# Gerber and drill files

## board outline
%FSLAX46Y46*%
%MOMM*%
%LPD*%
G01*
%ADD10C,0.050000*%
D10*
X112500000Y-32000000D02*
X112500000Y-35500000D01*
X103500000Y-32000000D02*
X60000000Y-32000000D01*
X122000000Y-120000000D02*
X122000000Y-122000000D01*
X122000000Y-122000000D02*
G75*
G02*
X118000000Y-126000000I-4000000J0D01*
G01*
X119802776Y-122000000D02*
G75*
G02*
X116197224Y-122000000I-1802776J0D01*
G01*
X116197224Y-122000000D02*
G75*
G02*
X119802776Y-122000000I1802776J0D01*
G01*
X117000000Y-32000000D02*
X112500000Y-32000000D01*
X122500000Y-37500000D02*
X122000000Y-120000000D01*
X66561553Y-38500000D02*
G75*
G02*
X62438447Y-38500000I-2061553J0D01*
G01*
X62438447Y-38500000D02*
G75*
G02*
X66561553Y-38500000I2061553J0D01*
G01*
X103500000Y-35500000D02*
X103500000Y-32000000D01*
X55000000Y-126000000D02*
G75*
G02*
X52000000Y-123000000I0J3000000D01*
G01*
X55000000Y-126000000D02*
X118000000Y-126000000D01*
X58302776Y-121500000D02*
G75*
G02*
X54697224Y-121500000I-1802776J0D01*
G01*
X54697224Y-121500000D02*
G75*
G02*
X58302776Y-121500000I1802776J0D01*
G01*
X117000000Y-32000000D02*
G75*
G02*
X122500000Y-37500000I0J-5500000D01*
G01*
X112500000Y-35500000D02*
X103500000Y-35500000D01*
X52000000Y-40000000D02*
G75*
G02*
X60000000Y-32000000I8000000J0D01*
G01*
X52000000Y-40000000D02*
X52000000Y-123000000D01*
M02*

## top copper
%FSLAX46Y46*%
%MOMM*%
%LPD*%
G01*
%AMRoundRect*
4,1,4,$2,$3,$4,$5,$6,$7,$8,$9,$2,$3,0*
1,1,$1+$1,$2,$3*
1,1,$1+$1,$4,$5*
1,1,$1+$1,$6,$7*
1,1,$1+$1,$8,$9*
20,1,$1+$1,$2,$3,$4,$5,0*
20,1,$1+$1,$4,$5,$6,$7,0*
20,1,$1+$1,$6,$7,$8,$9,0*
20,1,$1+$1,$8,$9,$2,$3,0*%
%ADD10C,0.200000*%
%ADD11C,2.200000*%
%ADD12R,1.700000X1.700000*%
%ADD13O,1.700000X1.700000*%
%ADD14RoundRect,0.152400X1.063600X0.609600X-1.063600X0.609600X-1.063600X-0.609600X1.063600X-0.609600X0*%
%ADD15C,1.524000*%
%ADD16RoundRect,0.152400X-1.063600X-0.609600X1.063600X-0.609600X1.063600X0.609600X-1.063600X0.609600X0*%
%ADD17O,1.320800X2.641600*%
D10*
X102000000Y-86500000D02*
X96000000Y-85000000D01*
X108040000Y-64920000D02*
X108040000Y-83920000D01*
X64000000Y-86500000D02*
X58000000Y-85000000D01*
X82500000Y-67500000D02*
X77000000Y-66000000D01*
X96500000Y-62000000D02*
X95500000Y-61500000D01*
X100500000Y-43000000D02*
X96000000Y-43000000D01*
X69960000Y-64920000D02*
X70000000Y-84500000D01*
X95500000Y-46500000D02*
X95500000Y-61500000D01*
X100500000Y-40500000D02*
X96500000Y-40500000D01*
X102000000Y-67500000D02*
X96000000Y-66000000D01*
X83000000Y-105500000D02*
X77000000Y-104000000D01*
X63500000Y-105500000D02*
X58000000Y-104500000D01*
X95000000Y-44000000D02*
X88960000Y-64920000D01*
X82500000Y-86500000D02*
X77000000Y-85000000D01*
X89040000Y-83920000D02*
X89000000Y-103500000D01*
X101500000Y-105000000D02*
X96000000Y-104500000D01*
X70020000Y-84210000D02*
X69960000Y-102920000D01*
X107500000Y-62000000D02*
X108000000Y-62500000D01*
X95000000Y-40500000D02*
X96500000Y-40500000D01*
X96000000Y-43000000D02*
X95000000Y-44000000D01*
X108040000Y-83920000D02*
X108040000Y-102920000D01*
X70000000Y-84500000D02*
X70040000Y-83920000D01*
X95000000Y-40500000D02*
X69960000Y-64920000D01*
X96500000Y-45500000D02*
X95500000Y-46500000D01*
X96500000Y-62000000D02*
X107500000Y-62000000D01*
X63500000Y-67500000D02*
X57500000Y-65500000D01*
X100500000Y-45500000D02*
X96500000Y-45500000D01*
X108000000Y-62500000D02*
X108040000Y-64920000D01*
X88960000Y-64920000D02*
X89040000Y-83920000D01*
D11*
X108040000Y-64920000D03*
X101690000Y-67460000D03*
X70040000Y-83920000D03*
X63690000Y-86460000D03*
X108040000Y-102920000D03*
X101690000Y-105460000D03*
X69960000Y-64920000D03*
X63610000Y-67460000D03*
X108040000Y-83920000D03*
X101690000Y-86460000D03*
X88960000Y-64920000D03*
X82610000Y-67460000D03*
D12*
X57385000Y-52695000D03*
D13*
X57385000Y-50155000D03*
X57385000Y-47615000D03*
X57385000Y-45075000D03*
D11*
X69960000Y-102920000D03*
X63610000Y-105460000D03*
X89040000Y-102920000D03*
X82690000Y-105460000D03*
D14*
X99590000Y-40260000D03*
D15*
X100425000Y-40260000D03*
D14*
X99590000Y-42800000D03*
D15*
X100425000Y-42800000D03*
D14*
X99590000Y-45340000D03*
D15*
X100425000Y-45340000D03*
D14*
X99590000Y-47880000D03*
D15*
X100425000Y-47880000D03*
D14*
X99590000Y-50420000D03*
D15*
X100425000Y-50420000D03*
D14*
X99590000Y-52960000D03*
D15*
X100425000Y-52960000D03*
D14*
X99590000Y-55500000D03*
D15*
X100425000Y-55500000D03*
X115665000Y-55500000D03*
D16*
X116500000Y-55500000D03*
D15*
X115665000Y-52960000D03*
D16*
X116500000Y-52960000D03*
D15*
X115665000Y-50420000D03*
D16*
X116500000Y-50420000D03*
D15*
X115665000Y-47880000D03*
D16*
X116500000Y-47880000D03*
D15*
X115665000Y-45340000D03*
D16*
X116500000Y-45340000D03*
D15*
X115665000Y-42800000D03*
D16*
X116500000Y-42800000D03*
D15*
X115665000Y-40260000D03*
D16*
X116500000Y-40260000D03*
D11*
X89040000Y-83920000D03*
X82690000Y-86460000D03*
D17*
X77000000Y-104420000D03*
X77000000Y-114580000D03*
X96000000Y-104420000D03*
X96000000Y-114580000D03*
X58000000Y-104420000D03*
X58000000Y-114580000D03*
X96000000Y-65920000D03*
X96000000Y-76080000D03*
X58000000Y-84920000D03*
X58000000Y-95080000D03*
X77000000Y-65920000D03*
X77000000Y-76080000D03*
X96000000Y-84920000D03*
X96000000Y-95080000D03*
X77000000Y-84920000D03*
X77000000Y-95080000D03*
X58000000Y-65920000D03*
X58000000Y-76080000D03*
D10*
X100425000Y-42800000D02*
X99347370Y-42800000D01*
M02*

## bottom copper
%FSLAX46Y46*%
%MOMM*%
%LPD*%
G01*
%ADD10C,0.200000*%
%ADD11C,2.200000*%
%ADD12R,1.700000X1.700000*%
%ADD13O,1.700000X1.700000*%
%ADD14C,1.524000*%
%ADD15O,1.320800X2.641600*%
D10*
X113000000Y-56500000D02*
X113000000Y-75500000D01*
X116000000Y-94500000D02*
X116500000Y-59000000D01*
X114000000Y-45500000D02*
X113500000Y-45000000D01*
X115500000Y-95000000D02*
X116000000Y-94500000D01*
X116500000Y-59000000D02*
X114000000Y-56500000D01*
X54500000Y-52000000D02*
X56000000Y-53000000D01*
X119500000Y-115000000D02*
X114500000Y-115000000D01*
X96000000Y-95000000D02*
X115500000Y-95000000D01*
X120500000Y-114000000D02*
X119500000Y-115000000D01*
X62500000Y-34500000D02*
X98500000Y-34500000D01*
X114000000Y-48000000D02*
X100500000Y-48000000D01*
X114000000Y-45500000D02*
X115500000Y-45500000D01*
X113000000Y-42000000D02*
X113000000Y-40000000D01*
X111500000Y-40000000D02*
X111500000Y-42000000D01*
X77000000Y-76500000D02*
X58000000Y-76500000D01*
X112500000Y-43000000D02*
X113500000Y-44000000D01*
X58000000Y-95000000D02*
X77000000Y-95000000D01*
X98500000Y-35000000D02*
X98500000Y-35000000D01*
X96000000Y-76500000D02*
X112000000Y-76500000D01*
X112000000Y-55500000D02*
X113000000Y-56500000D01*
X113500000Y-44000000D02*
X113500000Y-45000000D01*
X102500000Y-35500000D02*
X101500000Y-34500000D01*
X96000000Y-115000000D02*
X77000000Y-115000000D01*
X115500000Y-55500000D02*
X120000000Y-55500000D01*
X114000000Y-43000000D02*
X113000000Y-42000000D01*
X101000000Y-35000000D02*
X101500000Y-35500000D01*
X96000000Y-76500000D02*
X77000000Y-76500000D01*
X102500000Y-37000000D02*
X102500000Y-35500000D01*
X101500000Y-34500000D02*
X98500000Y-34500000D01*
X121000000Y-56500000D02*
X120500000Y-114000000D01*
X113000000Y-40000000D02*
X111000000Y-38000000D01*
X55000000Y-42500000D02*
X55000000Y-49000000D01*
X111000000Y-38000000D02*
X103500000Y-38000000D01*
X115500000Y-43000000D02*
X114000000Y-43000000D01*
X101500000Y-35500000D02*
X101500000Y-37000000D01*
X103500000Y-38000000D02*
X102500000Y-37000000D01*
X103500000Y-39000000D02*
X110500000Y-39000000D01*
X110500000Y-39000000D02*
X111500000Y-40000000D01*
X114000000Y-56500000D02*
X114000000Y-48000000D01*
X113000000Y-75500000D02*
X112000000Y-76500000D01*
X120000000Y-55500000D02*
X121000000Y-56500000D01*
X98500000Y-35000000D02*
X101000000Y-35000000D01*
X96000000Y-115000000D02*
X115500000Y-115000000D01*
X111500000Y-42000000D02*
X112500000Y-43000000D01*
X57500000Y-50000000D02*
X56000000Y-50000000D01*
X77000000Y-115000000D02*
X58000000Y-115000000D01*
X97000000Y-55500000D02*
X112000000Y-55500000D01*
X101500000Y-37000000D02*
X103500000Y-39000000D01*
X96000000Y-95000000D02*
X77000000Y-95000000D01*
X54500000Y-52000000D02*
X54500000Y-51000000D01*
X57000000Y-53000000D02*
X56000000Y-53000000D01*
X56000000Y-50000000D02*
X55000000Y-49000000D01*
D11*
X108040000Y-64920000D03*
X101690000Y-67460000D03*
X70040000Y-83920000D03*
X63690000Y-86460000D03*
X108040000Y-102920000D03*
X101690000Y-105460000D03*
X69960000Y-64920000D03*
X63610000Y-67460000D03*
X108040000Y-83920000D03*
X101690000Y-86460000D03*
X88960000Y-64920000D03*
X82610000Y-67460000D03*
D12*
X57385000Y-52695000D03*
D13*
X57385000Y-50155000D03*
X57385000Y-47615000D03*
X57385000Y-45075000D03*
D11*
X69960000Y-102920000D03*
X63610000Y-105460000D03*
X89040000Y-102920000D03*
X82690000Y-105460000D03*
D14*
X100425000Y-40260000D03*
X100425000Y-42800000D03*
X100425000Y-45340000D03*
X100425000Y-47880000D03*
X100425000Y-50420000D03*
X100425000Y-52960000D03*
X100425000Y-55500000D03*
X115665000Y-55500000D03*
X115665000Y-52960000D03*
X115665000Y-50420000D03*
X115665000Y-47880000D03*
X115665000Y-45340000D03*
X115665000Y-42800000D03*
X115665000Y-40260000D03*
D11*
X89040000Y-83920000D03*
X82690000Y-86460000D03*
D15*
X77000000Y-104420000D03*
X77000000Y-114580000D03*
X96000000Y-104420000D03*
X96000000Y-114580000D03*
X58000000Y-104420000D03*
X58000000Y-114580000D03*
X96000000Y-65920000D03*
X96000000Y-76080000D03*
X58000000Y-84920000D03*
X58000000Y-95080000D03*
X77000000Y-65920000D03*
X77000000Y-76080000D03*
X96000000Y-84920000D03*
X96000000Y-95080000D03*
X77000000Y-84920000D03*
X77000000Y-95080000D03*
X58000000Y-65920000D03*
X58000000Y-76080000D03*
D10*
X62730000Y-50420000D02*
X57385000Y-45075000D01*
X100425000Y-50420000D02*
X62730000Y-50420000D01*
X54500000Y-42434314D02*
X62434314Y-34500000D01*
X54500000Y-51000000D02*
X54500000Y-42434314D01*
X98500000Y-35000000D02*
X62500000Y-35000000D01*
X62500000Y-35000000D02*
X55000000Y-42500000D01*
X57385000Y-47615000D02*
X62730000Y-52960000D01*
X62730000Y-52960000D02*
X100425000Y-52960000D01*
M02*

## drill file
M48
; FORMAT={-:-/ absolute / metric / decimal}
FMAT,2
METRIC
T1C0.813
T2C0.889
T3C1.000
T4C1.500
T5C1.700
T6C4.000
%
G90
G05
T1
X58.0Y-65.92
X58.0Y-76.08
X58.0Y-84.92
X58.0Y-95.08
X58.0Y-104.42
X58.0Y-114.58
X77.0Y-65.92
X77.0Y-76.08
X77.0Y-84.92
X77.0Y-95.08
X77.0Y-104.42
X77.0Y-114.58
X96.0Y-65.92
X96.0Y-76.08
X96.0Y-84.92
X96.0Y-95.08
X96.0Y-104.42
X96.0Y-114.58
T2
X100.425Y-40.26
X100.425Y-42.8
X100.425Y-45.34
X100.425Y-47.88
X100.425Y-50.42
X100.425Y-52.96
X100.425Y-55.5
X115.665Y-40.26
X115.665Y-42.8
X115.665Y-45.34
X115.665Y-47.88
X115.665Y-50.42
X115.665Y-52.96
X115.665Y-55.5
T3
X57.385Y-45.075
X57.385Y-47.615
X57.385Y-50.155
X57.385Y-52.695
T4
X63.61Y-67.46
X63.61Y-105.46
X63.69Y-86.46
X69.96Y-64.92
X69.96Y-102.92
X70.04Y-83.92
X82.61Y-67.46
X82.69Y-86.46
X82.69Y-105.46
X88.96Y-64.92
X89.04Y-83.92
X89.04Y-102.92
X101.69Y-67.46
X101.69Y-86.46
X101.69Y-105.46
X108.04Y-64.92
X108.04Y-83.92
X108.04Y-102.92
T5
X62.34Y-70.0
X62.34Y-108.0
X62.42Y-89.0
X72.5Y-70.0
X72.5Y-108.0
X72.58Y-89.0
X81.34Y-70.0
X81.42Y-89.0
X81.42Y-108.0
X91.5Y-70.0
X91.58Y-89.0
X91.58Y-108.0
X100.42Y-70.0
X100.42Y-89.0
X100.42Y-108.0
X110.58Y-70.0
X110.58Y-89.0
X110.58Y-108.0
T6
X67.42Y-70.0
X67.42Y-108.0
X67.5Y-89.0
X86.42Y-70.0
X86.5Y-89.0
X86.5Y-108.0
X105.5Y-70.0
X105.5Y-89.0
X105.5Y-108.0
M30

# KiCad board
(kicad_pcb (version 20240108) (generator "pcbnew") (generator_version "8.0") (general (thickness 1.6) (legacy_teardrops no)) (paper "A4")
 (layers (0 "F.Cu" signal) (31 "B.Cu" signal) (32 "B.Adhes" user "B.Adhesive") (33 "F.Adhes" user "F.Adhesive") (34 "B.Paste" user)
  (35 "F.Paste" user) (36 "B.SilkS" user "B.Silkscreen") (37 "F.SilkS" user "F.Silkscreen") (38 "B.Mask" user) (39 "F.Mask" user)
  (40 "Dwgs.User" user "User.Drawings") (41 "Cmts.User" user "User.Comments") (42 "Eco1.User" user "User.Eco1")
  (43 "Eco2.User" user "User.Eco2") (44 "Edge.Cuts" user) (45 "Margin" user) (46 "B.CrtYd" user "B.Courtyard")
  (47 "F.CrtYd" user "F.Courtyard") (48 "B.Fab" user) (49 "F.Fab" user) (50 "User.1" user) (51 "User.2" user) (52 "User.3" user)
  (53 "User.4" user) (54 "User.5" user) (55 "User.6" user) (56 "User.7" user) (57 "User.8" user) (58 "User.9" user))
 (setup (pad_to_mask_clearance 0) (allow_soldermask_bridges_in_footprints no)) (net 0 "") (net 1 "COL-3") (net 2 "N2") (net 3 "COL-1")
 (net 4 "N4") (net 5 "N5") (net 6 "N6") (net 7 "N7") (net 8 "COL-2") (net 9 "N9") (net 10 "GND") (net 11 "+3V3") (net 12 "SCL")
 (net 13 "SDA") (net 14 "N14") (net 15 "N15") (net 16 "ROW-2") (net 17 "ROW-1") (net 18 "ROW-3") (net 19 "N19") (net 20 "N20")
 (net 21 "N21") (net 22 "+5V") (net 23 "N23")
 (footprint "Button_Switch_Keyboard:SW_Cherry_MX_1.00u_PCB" (layer "F.Cu") (at 108.04 64.92)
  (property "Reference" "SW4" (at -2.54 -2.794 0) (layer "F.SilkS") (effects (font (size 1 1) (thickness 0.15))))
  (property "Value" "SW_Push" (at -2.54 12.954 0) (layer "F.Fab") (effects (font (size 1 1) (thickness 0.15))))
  (pad "" np_thru_hole circle (at -7.62 5.08) (size 1.7 1.7) (drill 1.7) (layers "*.Cu" "*.Mask"))
  (pad "" np_thru_hole circle (at -2.54 5.08) (size 4 4) (drill 4) (layers "*.Cu" "*.Mask"))
  (pad "" np_thru_hole circle (at 2.54 5.08) (size 1.7 1.7) (drill 1.7) (layers "*.Cu" "*.Mask"))
  (pad "1" thru_hole circle (at 0 0) (size 2.2 2.2) (drill 1.5) (layers "*.Cu" "*.Mask") (remove_unused_layers no) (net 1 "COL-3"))
  (pad "2" thru_hole circle (at -6.35 2.54) (size 2.2 2.2) (drill 1.5) (layers "*.Cu" "*.Mask") (remove_unused_layers no) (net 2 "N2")))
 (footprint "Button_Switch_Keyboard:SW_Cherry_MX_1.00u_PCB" (layer "F.Cu") (at 70.04 83.92)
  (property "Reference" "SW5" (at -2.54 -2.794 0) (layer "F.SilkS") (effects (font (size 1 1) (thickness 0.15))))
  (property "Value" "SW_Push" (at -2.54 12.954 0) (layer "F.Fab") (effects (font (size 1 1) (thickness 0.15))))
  (pad "" np_thru_hole circle (at -7.62 5.08) (size 1.7 1.7) (drill 1.7) (layers "*.Cu" "*.Mask"))
  (pad "" np_thru_hole circle (at -2.54 5.08) (size 4 4) (drill 4) (layers "*.Cu" "*.Mask"))
  (pad "" np_thru_hole circle (at 2.54 5.08) (size 1.7 1.7) (drill 1.7) (layers "*.Cu" "*.Mask"))
  (pad "1" thru_hole circle (at 0 0) (size 2.2 2.2) (drill 1.5) (layers "*.Cu" "*.Mask") (remove_unused_layers no) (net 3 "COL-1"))
  (pad "2" thru_hole circle (at -6.35 2.54) (size 2.2 2.2) (drill 1.5) (layers "*.Cu" "*.Mask") (remove_unused_layers no) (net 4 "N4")))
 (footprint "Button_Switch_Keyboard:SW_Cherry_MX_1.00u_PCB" (layer "F.Cu") (at 108.04 102.92)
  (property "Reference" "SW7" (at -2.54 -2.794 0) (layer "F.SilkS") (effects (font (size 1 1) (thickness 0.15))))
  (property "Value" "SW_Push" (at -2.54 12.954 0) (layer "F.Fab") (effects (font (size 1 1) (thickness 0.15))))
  (pad "" np_thru_hole circle (at -7.62 5.08) (size 1.7 1.7) (drill 1.7) (layers "*.Cu" "*.Mask"))
  (pad "" np_thru_hole circle (at -2.54 5.08) (size 4 4) (drill 4) (layers "*.Cu" "*.Mask"))
  (pad "" np_thru_hole circle (at 2.54 5.08) (size 1.7 1.7) (drill 1.7) (layers "*.Cu" "*.Mask"))
  (pad "1" thru_hole circle (at 0 0) (size 2.2 2.2) (drill 1.5) (layers "*.Cu" "*.Mask") (remove_unused_layers no) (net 1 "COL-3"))
  (pad "2" thru_hole circle (at -6.35 2.54) (size 2.2 2.2) (drill 1.5) (layers "*.Cu" "*.Mask") (remove_unused_layers no) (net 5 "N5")))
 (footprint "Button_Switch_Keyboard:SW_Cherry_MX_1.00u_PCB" (layer "F.Cu") (at 69.96 64.92)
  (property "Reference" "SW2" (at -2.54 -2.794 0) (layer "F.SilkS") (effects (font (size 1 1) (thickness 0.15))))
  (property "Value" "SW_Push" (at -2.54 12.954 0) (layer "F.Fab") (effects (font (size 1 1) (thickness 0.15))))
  (pad "" np_thru_hole circle (at -7.62 5.08) (size 1.7 1.7) (drill 1.7) (layers "*.Cu" "*.Mask"))
  (pad "" np_thru_hole circle (at -2.54 5.08) (size 4 4) (drill 4) (layers "*.Cu" "*.Mask"))
  (pad "" np_thru_hole circle (at 2.54 5.08) (size 1.7 1.7) (drill 1.7) (layers "*.Cu" "*.Mask"))
  (pad "1" thru_hole circle (at 0 0) (size 2.2 2.2) (drill 1.5) (layers "*.Cu" "*.Mask") (remove_unused_layers no) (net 3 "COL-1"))
  (pad "2" thru_hole circle (at -6.35 2.54) (size 2.2 2.2) (drill 1.5) (layers "*.Cu" "*.Mask") (remove_unused_layers no) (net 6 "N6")))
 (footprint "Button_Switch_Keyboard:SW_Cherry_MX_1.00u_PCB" (layer "F.Cu") (at 108.04 83.92)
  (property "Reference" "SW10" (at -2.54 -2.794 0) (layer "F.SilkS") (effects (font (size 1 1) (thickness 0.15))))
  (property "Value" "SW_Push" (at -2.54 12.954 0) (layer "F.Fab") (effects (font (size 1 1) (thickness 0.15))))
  (pad "" np_thru_hole circle (at -7.62 5.08) (size 1.7 1.7) (drill 1.7) (layers "*.Cu" "*.Mask"))
  (pad "" np_thru_hole circle (at -2.54 5.08) (size 4 4) (drill 4) (layers "*.Cu" "*.Mask"))
  (pad "" np_thru_hole circle (at 2.54 5.08) (size 1.7 1.7) (drill 1.7) (layers "*.Cu" "*.Mask"))
  (pad "1" thru_hole circle (at 0 0) (size 2.2 2.2) (drill 1.5) (layers "*.Cu" "*.Mask") (remove_unused_layers no) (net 1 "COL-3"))
  (pad "2" thru_hole circle (at -6.35 2.54) (size 2.2 2.2) (drill 1.5) (layers "*.Cu" "*.Mask") (remove_unused_layers no) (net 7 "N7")))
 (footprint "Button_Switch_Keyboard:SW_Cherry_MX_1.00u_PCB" (layer "F.Cu") (at 88.96 64.92)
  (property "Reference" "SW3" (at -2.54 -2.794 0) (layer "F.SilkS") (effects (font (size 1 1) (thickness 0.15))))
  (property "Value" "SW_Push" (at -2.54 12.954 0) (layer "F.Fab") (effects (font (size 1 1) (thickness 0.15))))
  (pad "" np_thru_hole circle (at -7.62 5.08) (size 1.7 1.7) (drill 1.7) (layers "*.Cu" "*.Mask"))
  (pad "" np_thru_hole circle (at -2.54 5.08) (size 4 4) (drill 4) (layers "*.Cu" "*.Mask"))
  (pad "" np_thru_hole circle (at 2.54 5.08) (size 1.7 1.7) (drill 1.7) (layers "*.Cu" "*.Mask"))
  (pad "1" thru_hole circle (at 0 0) (size 2.2 2.2) (drill 1.5) (layers "*.Cu" "*.Mask") (remove_unused_layers no) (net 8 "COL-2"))
  (pad "2" thru_hole circle (at -6.35 2.54) (size 2.2 2.2) (drill 1.5) (layers "*.Cu" "*.Mask") (remove_unused_layers no) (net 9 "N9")))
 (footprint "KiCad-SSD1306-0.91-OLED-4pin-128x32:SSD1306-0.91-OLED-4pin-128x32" (layer "F.Cu") (at 93.885 54.885 180)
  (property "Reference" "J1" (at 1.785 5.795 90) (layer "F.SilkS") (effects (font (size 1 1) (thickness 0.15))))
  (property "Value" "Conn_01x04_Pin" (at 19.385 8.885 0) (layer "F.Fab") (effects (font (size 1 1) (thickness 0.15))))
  (pad "1" thru_hole rect (at 36.5 2.19 180) (size 1.7 1.7) (drill 1) (layers "*.Cu" "*.Mask") (remove_unused_layers no) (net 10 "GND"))
  (pad "2" thru_hole oval (at 36.5 4.73 180) (size 1.7 1.7) (drill 1) (layers "*.Cu" "*.Mask") (remove_unused_layers no) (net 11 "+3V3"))
  (pad "3" thru_hole oval (at 36.5 7.27 180) (size 1.7 1.7) (drill 1) (layers "*.Cu" "*.Mask") (remove_unused_layers no) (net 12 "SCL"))
  (pad "4" thru_hole oval (at 36.5 9.81 180) (size 1.7 1.7) (drill 1) (layers "*.Cu" "*.Mask") (remove_unused_layers no) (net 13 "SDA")))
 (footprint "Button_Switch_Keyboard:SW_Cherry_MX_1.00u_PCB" (layer "F.Cu") (at 69.96 102.92)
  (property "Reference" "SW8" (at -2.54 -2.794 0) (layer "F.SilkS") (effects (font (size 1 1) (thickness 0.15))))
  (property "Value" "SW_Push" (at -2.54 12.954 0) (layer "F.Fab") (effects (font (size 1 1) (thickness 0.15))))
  (pad "" np_thru_hole circle (at -7.62 5.08) (size 1.7 1.7) (drill 1.7) (layers "*.Cu" "*.Mask"))
  (pad "" np_thru_hole circle (at -2.54 5.08) (size 4 4) (drill 4) (layers "*.Cu" "*.Mask"))
  (pad "" np_thru_hole circle (at 2.54 5.08) (size 1.7 1.7) (drill 1.7) (layers "*.Cu" "*.Mask"))
  (pad "1" thru_hole circle (at 0 0) (size 2.2 2.2) (drill 1.5) (layers "*.Cu" "*.Mask") (remove_unused_layers no) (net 3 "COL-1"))
  (pad "2" thru_hole circle (at -6.35 2.54) (size 2.2 2.2) (drill 1.5) (layers "*.Cu" "*.Mask") (remove_unused_layers no) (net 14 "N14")))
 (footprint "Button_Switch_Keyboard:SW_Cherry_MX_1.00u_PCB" (layer "F.Cu") (at 89.04 102.92)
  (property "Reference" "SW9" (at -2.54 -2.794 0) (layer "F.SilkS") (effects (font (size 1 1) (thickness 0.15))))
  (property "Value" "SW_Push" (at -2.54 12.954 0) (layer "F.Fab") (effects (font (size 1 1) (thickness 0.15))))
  (pad "" np_thru_hole circle (at -7.62 5.08) (size 1.7 1.7) (drill 1.7) (layers "*.Cu" "*.Mask"))
  (pad "" np_thru_hole circle (at -2.54 5.08) (size 4 4) (drill 4) (layers "*.Cu" "*.Mask"))
  (pad "" np_thru_hole circle (at 2.54 5.08) (size 1.7 1.7) (drill 1.7) (layers "*.Cu" "*.Mask"))
  (pad "1" thru_hole circle (at 0 0) (size 2.2 2.2) (drill 1.5) (layers "*.Cu" "*.Mask") (remove_unused_layers no) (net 8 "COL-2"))
  (pad "2" thru_hole circle (at -6.35 2.54) (size 2.2 2.2) (drill 1.5) (layers "*.Cu" "*.Mask") (remove_unused_layers no) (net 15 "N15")))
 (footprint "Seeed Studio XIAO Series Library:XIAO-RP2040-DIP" (layer "F.Cu") (at 108.045 47.88)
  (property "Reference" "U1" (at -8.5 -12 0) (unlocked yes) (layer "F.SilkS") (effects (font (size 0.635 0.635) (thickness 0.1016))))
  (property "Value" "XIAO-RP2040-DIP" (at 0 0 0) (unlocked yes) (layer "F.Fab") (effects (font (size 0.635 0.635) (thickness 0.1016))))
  (pad "1" smd roundrect (at -8.455 -7.62 180) (size 2.432 1.524) (layers "F.Cu" "F.Mask") (roundrect_rratio 0.1) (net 3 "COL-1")
   (thermal_bridge_angle 45))
  (pad "1" thru_hole circle (at -7.62 -7.62 180) (size 1.524 1.524) (drill 0.889) (layers "*.Cu" "*.Mask") (remove_unused_layers no)
   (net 3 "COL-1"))
  (pad "2" smd roundrect (at -8.455 -5.08 180) (size 2.432 1.524) (layers "F.Cu" "F.Mask") (roundrect_rratio 0.1) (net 8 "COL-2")
   (thermal_bridge_angle 45))
  (pad "2" thru_hole circle (at -7.62 -5.08 180) (size 1.524 1.524) (drill 0.889) (layers "*.Cu" "*.Mask") (remove_unused_layers no)
   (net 8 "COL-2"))
  (pad "3" smd roundrect (at -8.455 -2.54 180) (size 2.432 1.524) (layers "F.Cu" "F.Mask") (roundrect_rratio 0.1) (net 1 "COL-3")
   (thermal_bridge_angle 45))
  (pad "3" thru_hole circle (at -7.62 -2.54 180) (size 1.524 1.524) (drill 0.889) (layers "*.Cu" "*.Mask") (remove_unused_layers no)
   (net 1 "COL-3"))
  (pad "4" smd roundrect (at -8.455 0 180) (size 2.432 1.524) (layers "F.Cu" "F.Mask") (roundrect_rratio 0.1) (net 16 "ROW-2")
   (thermal_bridge_angle 45))
  (pad "4" thru_hole circle (at -7.62 0 180) (size 1.524 1.524) (drill 0.889) (layers "*.Cu" "*.Mask") (remove_unused_layers no)
   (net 16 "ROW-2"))
  (pad "5" smd roundrect (at -8.455 2.54 180) (size 2.432 1.524) (layers "F.Cu" "F.Mask") (roundrect_rratio 0.1) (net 13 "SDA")
   (thermal_bridge_angle 45))
  (pad "5" thru_hole circle (at -7.62 2.54 180) (size 1.524 1.524) (drill 0.889) (layers "*.Cu" "*.Mask") (remove_unused_layers no)
   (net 13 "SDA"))
  (pad "6" smd roundrect (at -8.455 5.08 180) (size 2.432 1.524) (layers "F.Cu" "F.Mask") (roundrect_rratio 0.1) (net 12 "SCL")
   (thermal_bridge_angle 45))
  (pad "6" thru_hole circle (at -7.62 5.08 180) (size 1.524 1.524) (drill 0.889) (layers "*.Cu" "*.Mask") (remove_unused_layers no)
   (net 12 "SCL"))
  (pad "7" smd roundrect (at -8.455 7.62 180) (size 2.432 1.524) (layers "F.Cu" "F.Mask") (roundrect_rratio 0.1) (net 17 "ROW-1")
   (thermal_bridge_angle 45))
  (pad "7" thru_hole circle (at -7.62 7.62 180) (size 1.524 1.524) (drill 0.889) (layers "*.Cu" "*.Mask") (remove_unused_layers no)
   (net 17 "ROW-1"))
  (pad "8" thru_hole circle (at 7.62 7.62) (size 1.524 1.524) (drill 0.889) (layers "*.Cu" "*.Mask") (remove_unused_layers no)
   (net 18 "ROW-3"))
  (pad "8" smd roundrect (at 8.455 7.62) (size 2.432 1.524) (layers "F.Cu" "F.Mask") (roundrect_rratio 0.1) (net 18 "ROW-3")
   (thermal_bridge_angle 45))
  (pad "9" thru_hole circle (at 7.62 5.08) (size 1.524 1.524) (drill 0.889) (layers "*.Cu" "*.Mask") (remove_unused_layers no)
   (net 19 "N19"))
  (pad "9" smd roundrect (at 8.455 5.08) (size 2.432 1.524) (layers "F.Cu" "F.Mask") (roundrect_rratio 0.1) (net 19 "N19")
   (thermal_bridge_angle 45))
  (pad "10" thru_hole circle (at 7.62 2.54) (size 1.524 1.524) (drill 0.889) (layers "*.Cu" "*.Mask") (remove_unused_layers no)
   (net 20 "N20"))
  (pad "10" smd roundrect (at 8.455 2.54) (size 2.432 1.524) (layers "F.Cu" "F.Mask") (roundrect_rratio 0.1) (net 20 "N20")
   (thermal_bridge_angle 45))
  (pad "11" thru_hole circle (at 7.62 0) (size 1.524 1.524) (drill 0.889) (layers "*.Cu" "*.Mask") (remove_unused_layers no) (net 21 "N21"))
  (pad "11" smd roundrect (at 8.455 0) (size 2.432 1.524) (layers "F.Cu" "F.Mask") (roundrect_rratio 0.1) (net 21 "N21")
   (thermal_bridge_angle 45))
  (pad "12" thru_hole circle (at 7.62 -2.54) (size 1.524 1.524) (drill 0.889) (layers "*.Cu" "*.Mask") (remove_unused_layers no)
   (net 11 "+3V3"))
  (pad "12" smd roundrect (at 8.455 -2.54) (size 2.432 1.524) (layers "F.Cu" "F.Mask") (roundrect_rratio 0.1) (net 11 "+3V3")
   (thermal_bridge_angle 45))
  (pad "13" thru_hole circle (at 7.62 -5.08) (size 1.524 1.524) (drill 0.889) (layers "*.Cu" "*.Mask") (remove_unused_layers no)
   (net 10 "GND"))
  (pad "13" smd roundrect (at 8.455 -5.08) (size 2.432 1.524) (layers "F.Cu" "F.Mask") (roundrect_rratio 0.1) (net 10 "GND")
   (thermal_bridge_angle 45))
  (pad "14" thru_hole circle (at 7.62 -7.62) (size 1.524 1.524) (drill 0.889) (layers "*.Cu" "*.Mask") (remove_unused_layers no)
   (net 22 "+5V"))
  (pad "14" smd roundrect (at 8.455 -7.62) (size 2.432 1.524) (layers "F.Cu" "F.Mask") (roundrect_rratio 0.1) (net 22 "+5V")
   (thermal_bridge_angle 45)))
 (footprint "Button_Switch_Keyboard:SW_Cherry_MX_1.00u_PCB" (layer "F.Cu") (at 89.04 83.92)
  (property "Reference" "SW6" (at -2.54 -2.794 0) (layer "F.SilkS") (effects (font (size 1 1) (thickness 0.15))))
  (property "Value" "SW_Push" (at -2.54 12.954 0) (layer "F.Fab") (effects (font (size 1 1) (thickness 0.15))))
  (pad "" np_thru_hole circle (at -7.62 5.08) (size 1.7 1.7) (drill 1.7) (layers "*.Cu" "*.Mask"))
  (pad "" np_thru_hole circle (at -2.54 5.08) (size 4 4) (drill 4) (layers "*.Cu" "*.Mask"))
  (pad "" np_thru_hole circle (at 2.54 5.08) (size 1.7 1.7) (drill 1.7) (layers "*.Cu" "*.Mask"))
  (pad "1" thru_hole circle (at 0 0) (size 2.2 2.2) (drill 1.5) (layers "*.Cu" "*.Mask") (remove_unused_layers no) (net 8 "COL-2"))
  (pad "2" thru_hole circle (at -6.35 2.54) (size 2.2 2.2) (drill 1.5) (layers "*.Cu" "*.Mask") (remove_unused_layers no) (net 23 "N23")))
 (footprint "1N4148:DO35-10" (layer "B.Cu") (at 77 109.5 90)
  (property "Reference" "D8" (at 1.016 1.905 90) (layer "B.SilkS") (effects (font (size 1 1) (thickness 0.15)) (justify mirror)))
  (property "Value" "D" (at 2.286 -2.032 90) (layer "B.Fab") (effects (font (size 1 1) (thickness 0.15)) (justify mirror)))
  (pad "A" thru_hole oval (at 5.08 0 90) (size 2.6416 1.3208) (drill 0.8128) (layers "*.Cu" "*.Mask") (remove_unused_layers no)
   (solder_mask_margin 0.102))
  (pad "C" thru_hole oval (at -5.08 0 90) (size 2.6416 1.3208) (drill 0.8128) (layers "*.Cu" "*.Mask") (remove_unused_layers no)
   (solder_mask_margin 0.102)))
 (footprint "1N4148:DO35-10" (layer "B.Cu") (at 96 109.5 90)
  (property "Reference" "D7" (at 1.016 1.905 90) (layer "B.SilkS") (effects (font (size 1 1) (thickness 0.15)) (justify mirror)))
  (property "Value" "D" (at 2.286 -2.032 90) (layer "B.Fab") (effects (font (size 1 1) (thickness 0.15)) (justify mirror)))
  (pad "A" thru_hole oval (at 5.08 0 90) (size 2.6416 1.3208) (drill 0.8128) (layers "*.Cu" "*.Mask") (remove_unused_layers no)
   (solder_mask_margin 0.102))
  (pad "C" thru_hole oval (at -5.08 0 90) (size 2.6416 1.3208) (drill 0.8128) (layers "*.Cu" "*.Mask") (remove_unused_layers no)
   (solder_mask_margin 0.102)))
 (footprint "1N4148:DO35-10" (layer "B.Cu") (at 58 109.5 90)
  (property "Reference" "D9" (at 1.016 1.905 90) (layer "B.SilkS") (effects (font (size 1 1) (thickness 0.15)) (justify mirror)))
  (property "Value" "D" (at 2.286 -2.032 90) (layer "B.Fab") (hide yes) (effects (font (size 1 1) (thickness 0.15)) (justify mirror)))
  (pad "A" thru_hole oval (at 5.08 0 90) (size 2.6416 1.3208) (drill 0.8128) (layers "*.Cu" "*.Mask") (remove_unused_layers no)
   (solder_mask_margin 0.102))
  (pad "C" thru_hole oval (at -5.08 0 90) (size 2.6416 1.3208) (drill 0.8128) (layers "*.Cu" "*.Mask") (remove_unused_layers no)
   (solder_mask_margin 0.102)))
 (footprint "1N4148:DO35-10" (layer "B.Cu") (at 96 71 90)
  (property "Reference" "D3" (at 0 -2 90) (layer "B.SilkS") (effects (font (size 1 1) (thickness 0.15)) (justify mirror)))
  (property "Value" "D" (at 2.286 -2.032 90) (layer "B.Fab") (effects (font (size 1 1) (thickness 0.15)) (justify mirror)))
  (pad "A" thru_hole oval (at 5.08 0 90) (size 2.6416 1.3208) (drill 0.8128) (layers "*.Cu" "*.Mask") (remove_unused_layers no)
   (solder_mask_margin 0.102))
  (pad "C" thru_hole oval (at -5.08 0 90) (size 2.6416 1.3208) (drill 0.8128) (layers "*.Cu" "*.Mask") (remove_unused_layers no)
   (solder_mask_margin 0.102)))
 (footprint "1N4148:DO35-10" (layer "B.Cu") (at 58 90 90)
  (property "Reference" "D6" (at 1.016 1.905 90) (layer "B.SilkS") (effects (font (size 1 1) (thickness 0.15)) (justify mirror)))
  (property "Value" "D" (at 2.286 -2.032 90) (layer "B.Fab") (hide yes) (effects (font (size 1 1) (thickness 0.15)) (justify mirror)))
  (pad "A" thru_hole oval (at 5.08 0 90) (size 2.6416 1.3208) (drill 0.8128) (layers "*.Cu" "*.Mask") (remove_unused_layers no)
   (solder_mask_margin 0.102))
  (pad "C" thru_hole oval (at -5.08 0 90) (size 2.6416 1.3208) (drill 0.8128) (layers "*.Cu" "*.Mask") (remove_unused_layers no)
   (solder_mask_margin 0.102)))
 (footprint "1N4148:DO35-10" (layer "B.Cu") (at 77 71 90)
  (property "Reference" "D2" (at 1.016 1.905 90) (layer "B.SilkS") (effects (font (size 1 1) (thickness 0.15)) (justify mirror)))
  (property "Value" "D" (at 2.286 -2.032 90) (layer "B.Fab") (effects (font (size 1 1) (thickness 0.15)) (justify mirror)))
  (pad "A" thru_hole oval (at 5.08 0 90) (size 2.6416 1.3208) (drill 0.8128) (layers "*.Cu" "*.Mask") (remove_unused_layers no)
   (solder_mask_margin 0.102))
  (pad "C" thru_hole oval (at -5.08 0 90) (size 2.6416 1.3208) (drill 0.8128) (layers "*.Cu" "*.Mask") (remove_unused_layers no)
   (solder_mask_margin 0.102)))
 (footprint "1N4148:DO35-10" (layer "B.Cu") (at 96 90 90)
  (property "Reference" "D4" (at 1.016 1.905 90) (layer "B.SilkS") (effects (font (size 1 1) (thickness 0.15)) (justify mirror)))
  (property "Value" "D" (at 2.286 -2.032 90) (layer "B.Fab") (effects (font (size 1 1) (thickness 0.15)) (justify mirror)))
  (pad "A" thru_hole oval (at 5.08 0 90) (size 2.6416 1.3208) (drill 0.8128) (layers "*.Cu" "*.Mask") (remove_unused_layers no)
   (solder_mask_margin 0.102))
  (pad "C" thru_hole oval (at -5.08 0 90) (size 2.6416 1.3208) (drill 0.8128) (layers "*.Cu" "*.Mask") (remove_unused_layers no)
   (solder_mask_margin 0.102)))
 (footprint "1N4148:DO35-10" (layer "B.Cu") (at 77 90 90)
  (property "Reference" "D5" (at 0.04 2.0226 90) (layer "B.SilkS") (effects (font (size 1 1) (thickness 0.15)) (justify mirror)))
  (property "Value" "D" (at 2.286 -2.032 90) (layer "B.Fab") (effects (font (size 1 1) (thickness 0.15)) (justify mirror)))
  (pad "A" thru_hole oval (at 5.08 0 90) (size 2.6416 1.3208) (drill 0.8128) (layers "*.Cu" "*.Mask") (remove_unused_layers no)
   (solder_mask_margin 0.102))
  (pad "C" thru_hole oval (at -5.08 0 90) (size 2.6416 1.3208) (drill 0.8128) (layers "*.Cu" "*.Mask") (remove_unused_layers no)
   (solder_mask_margin 0.102)))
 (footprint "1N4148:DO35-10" (layer "B.Cu") (at 58 71 90)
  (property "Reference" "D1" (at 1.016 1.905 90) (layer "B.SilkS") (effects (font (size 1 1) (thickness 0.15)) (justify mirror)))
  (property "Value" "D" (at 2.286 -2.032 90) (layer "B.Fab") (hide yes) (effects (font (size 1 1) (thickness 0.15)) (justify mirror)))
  (pad "A" thru_hole oval (at 5.08 0 90) (size 2.6416 1.3208) (drill 0.8128) (layers "*.Cu" "*.Mask") (remove_unused_layers no)
   (solder_mask_margin 0.102))
  (pad "C" thru_hole oval (at -5.08 0 90) (size 2.6416 1.3208) (drill 0.8128) (layers "*.Cu" "*.Mask") (remove_unused_layers no)
   (solder_mask_margin 0.102)))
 (gr_line (start 102 86.5) (end 96 85) (stroke (width 0.2) (type default)) (layer "F.Cu") (net 7))
 (gr_line (start 108.04 64.92) (end 108.04 83.92) (stroke (width 0.2) (type default)) (layer "F.Cu") (net 1))
 (gr_line (start 64 86.5) (end 58 85) (stroke (width 0.2) (type default)) (layer "F.Cu") (net 4))
 (gr_line (start 82.5 67.5) (end 77 66) (stroke (width 0.2) (type default)) (layer "F.Cu") (net 9))
 (gr_line (start 96.5 62) (end 95.5 61.5) (stroke (width 0.2) (type default)) (layer "F.Cu") (net 1))
 (gr_line (start 100.5 43) (end 96 43) (stroke (width 0.2) (type default)) (layer "F.Cu") (net 8))
 (gr_line (start 69.96 64.92) (end 70 84.5) (stroke (width 0.2) (type default)) (layer "F.Cu") (net 3))
 (gr_line (start 95.5 46.5) (end 95.5 61.5) (stroke (width 0.2) (type default)) (layer "F.Cu") (net 1))
 (gr_line (start 100.5 40.5) (end 96.5 40.5) (stroke (width 0.2) (type default)) (layer "F.Cu") (net 3))
 (gr_line (start 102 67.5) (end 96 66) (stroke (width 0.2) (type default)) (layer "F.Cu") (net 2))
 (gr_line (start 83 105.5) (end 77 104) (stroke (width 0.2) (type default)) (layer "F.Cu") (net 15))
 (gr_line (start 63.5 105.5) (end 58 104.5) (stroke (width 0.2) (type default)) (layer "F.Cu") (net 14))
 (gr_line (start 95 44) (end 88.96 64.92) (stroke (width 0.2) (type default)) (layer "F.Cu") (net 8))
 (gr_line (start 82.5 86.5) (end 77 85) (stroke (width 0.2) (type default)) (layer "F.Cu") (net 23))
 (gr_line (start 89.04 83.92) (end 89 103.5) (stroke (width 0.2) (type default)) (layer "F.Cu") (net 8))
 (gr_line (start 101.5 105) (end 96 104.5) (stroke (width 0.2) (type default)) (layer "F.Cu") (net 5))
 (gr_line (start 70.02 84.21) (end 69.96 102.92) (stroke (width 0.2) (type default)) (layer "F.Cu") (net 3))
 (gr_line (start 107.5 62) (end 108 62.5) (stroke (width 0.2) (type default)) (layer "F.Cu") (net 1))
 (gr_line (start 95 40.5) (end 96.5 40.5) (stroke (width 0.2) (type default)) (layer "F.Cu") (net 3))
 (gr_line (start 96 43) (end 95 44) (stroke (width 0.2) (type default)) (layer "F.Cu") (net 8))
 (gr_line (start 108.04 83.92) (end 108.04 102.92) (stroke (width 0.2) (type default)) (layer "F.Cu") (net 1))
 (gr_line (start 70 84.5) (end 70.04 83.92) (stroke (width 0.2) (type default)) (layer "F.Cu") (net 3))
 (gr_line (start 95 40.5) (end 69.96 64.92) (stroke (width 0.2) (type default)) (layer "F.Cu") (net 3))
 (gr_line (start 96.5 45.5) (end 95.5 46.5) (stroke (width 0.2) (type default)) (layer "F.Cu") (net 1))
 (gr_line (start 96.5 62) (end 107.5 62) (stroke (width 0.2) (type default)) (layer "F.Cu") (net 1))
 (gr_line (start 63.5 67.5) (end 57.5 65.5) (stroke (width 0.2) (type default)) (layer "F.Cu") (net 6))
 (gr_line (start 100.5 45.5) (end 96.5 45.5) (stroke (width 0.2) (type default)) (layer "F.Cu") (net 1))
 (gr_line (start 108 62.5) (end 108.04 64.92) (stroke (width 0.2) (type default)) (layer "F.Cu") (net 1))
 (gr_line (start 88.96 64.92) (end 89.04 83.92) (stroke (width 0.2) (type default)) (layer "F.Cu") (net 8))
 (gr_line (start 113 56.5) (end 113 75.5) (stroke (width 0.2) (type default)) (layer "B.Cu") (net 17))
 (gr_line (start 116 94.5) (end 116.5 59) (stroke (width 0.2) (type default)) (layer "B.Cu") (net 16))
 (gr_line (start 114 45.5) (end 113.5 45) (stroke (width 0.2) (type default)) (layer "B.Cu") (net 11))
 (gr_line (start 115.5 95) (end 116 94.5) (stroke (width 0.2) (type default)) (layer "B.Cu") (net 16))
 (gr_line (start 116.5 59) (end 114 56.5) (stroke (width 0.2) (type default)) (layer "B.Cu") (net 16))
 (gr_line (start 54.5 52) (end 56 53) (stroke (width 0.2) (type default)) (layer "B.Cu") (net 10))
 (gr_line (start 119.5 115) (end 114.5 115) (stroke (width 0.2) (type default)) (layer "B.Cu") (net 18))
 (gr_line (start 96 95) (end 115.5 95) (stroke (width 0.2) (type default)) (layer "B.Cu") (net 16))
 (gr_line (start 120.5 114) (end 119.5 115) (stroke (width 0.2) (type default)) (layer "B.Cu") (net 18))
 (gr_line (start 62.5 34.5) (end 98.5 34.5) (stroke (width 0.2) (type default)) (layer "B.Cu") (net 10))
 (gr_line (start 114 48) (end 100.5 48) (stroke (width 0.2) (type default)) (layer "B.Cu") (net 16))
 (gr_line (start 114 45.5) (end 115.5 45.5) (stroke (width 0.2) (type default)) (layer "B.Cu") (net 11))
 (gr_line (start 113 42) (end 113 40) (stroke (width 0.2) (type default)) (layer "B.Cu") (net 10))
 (gr_line (start 111.5 40) (end 111.5 42) (stroke (width 0.2) (type default)) (layer "B.Cu") (net 11))
 (gr_line (start 77 76.5) (end 58 76.5) (stroke (width 0.2) (type default)) (layer "B.Cu") (net 17))
 (gr_line (start 112.5 43) (end 113.5 44) (stroke (width 0.2) (type default)) (layer "B.Cu") (net 11))
 (gr_line (start 58 95) (end 77 95) (stroke (width 0.2) (type default)) (layer "B.Cu") (net 16))
 (gr_line (start 98.5 35) (end 98.5 35) (stroke (width 0.2) (type default)) (layer "B.Cu") (net 11))
 (gr_line (start 96 76.5) (end 112 76.5) (stroke (width 0.2) (type default)) (layer "B.Cu") (net 17))
 (gr_line (start 112 55.5) (end 113 56.5) (stroke (width 0.2) (type default)) (layer "B.Cu") (net 17))
 (gr_line (start 113.5 44) (end 113.5 45) (stroke (width 0.2) (type default)) (layer "B.Cu") (net 11))
 (gr_line (start 102.5 35.5) (end 101.5 34.5) (stroke (width 0.2) (type default)) (layer "B.Cu") (net 10))
 (gr_line (start 96 115) (end 77 115) (stroke (width 0.2) (type default)) (layer "B.Cu") (net 18))
 (gr_line (start 115.5 55.5) (end 120 55.5) (stroke (width 0.2) (type default)) (layer "B.Cu") (net 18))
 (gr_line (start 114 43) (end 113 42) (stroke (width 0.2) (type default)) (layer "B.Cu") (net 10))
 (gr_line (start 101 35) (end 101.5 35.5) (stroke (width 0.2) (type default)) (layer "B.Cu") (net 11))
 (gr_line (start 96 76.5) (end 77 76.5) (stroke (width 0.2) (type default)) (layer "B.Cu") (net 17))
 (gr_line (start 102.5 37) (end 102.5 35.5) (stroke (width 0.2) (type default)) (layer "B.Cu") (net 10))
 (gr_line (start 101.5 34.5) (end 98.5 34.5) (stroke (width 0.2) (type default)) (layer "B.Cu") (net 10))
 (gr_line (start 121 56.5) (end 120.5 114) (stroke (width 0.2) (type default)) (layer "B.Cu") (net 18))
 (gr_line (start 113 40) (end 111 38) (stroke (width 0.2) (type default)) (layer "B.Cu") (net 10))
 (gr_line (start 55 42.5) (end 55 49) (stroke (width 0.2) (type default)) (layer "B.Cu") (net 11))
 (gr_line (start 111 38) (end 103.5 38) (stroke (width 0.2) (type default)) (layer "B.Cu") (net 10))
 (gr_line (start 115.5 43) (end 114 43) (stroke (width 0.2) (type default)) (layer "B.Cu") (net 10))
 (gr_line (start 101.5 35.5) (end 101.5 37) (stroke (width 0.2) (type default)) (layer "B.Cu") (net 11))
 (gr_line (start 103.5 38) (end 102.5 37) (stroke (width 0.2) (type default)) (layer "B.Cu") (net 10))
 (gr_line (start 103.5 39) (end 110.5 39) (stroke (width 0.2) (type default)) (layer "B.Cu") (net 11))
 (gr_line (start 110.5 39) (end 111.5 40) (stroke (width 0.2) (type default)) (layer "B.Cu") (net 11))
 (gr_line (start 114 56.5) (end 114 48) (stroke (width 0.2) (type default)) (layer "B.Cu") (net 16))
 (gr_line (start 113 75.5) (end 112 76.5) (stroke (width 0.2) (type default)) (layer "B.Cu") (net 17))
 (gr_line (start 120 55.5) (end 121 56.5) (stroke (width 0.2) (type default)) (layer "B.Cu") (net 18))
 (gr_line (start 98.5 35) (end 101 35) (stroke (width 0.2) (type default)) (layer "B.Cu") (net 11))
 (gr_line (start 96 115) (end 115.5 115) (stroke (width 0.2) (type default)) (layer "B.Cu") (net 18))
 (gr_line (start 111.5 42) (end 112.5 43) (stroke (width 0.2) (type default)) (layer "B.Cu") (net 11))
 (gr_line (start 57.5 50) (end 56 50) (stroke (width 0.2) (type default)) (layer "B.Cu") (net 11))
 (gr_line (start 77 115) (end 58 115) (stroke (width 0.2) (type default)) (layer "B.Cu") (net 18))
 (gr_line (start 97 55.5) (end 112 55.5) (stroke (width 0.2) (type default)) (layer "B.Cu") (net 17))
 (gr_line (start 101.5 37) (end 103.5 39) (stroke (width 0.2) (type default)) (layer "B.Cu") (net 11))
 (gr_line (start 96 95) (end 77 95) (stroke (width 0.2) (type default)) (layer "B.Cu") (net 16))
 (gr_line (start 54.5 52) (end 54.5 51) (stroke (width 0.2) (type default)) (layer "B.Cu") (net 10))
 (gr_line (start 57 53) (end 56 53) (stroke (width 0.2) (type default)) (layer "B.Cu") (net 10))
 (gr_line (start 56 50) (end 55 49) (stroke (width 0.2) (type default)) (layer "B.Cu") (net 11))
 (gr_line (start 112.5 32) (end 112.5 35.5) (stroke (width 0.05) (type default)) (layer "Edge.Cuts"))
 (gr_line (start 103.5 32) (end 60 32) (stroke (width 0.05) (type default)) (layer "Edge.Cuts"))
 (gr_line (start 122 120) (end 122 122) (stroke (width 0.05) (type default)) (layer "Edge.Cuts"))
 (gr_arc (start 122 122) (mid 120.828427 124.828427) (end 118 126) (stroke (width 0.05) (type default)) (layer "Edge.Cuts"))
 (gr_circle (center 118 122) (end 119.5 121) (stroke (width 0.05) (type default)) (fill none) (layer "Edge.Cuts"))
 (gr_line (start 117 32) (end 112.5 32) (stroke (width 0.05) (type default)) (layer "Edge.Cuts"))
 (gr_line (start 122.5 37.5) (end 122 120) (stroke (width 0.05) (type default)) (layer "Edge.Cuts"))
 (gr_circle (center 64.5 38.5) (end 66.5 38) (stroke (width 0.05) (type default)) (fill none) (layer "Edge.Cuts"))
 (gr_line (start 103.5 35.5) (end 103.5 32) (stroke (width 0.05) (type default)) (layer "Edge.Cuts"))
 (gr_arc (start 55 126) (mid 52.87868 125.12132) (end 52 123) (stroke (width 0.05) (type default)) (layer "Edge.Cuts"))
 (gr_line (start 55 126) (end 118 126) (stroke (width 0.05) (type default)) (layer "Edge.Cuts"))
 (gr_circle (center 56.5 121.5) (end 58 120.5) (stroke (width 0.05) (type default)) (fill none) (layer "Edge.Cuts"))
 (gr_arc (start 117 32) (mid 120.889087 33.610913) (end 122.5 37.5) (stroke (width 0.05) (type default)) (layer "Edge.Cuts"))
 (gr_line (start 112.5 35.5) (end 103.5 35.5) (stroke (width 0.05) (type default)) (layer "Edge.Cuts"))
 (gr_arc (start 52 40) (mid 54.343146 34.343146) (end 60 32) (stroke (width 0.05) (type default)) (layer "Edge.Cuts"))
 (gr_line (start 52 40) (end 52 123) (stroke (width 0.05) (type default)) (layer "Edge.Cuts"))
 (segment (start 62.73 50.42) (end 57.385 45.075) (width 0.2) (layer "B.Cu") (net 13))
 (segment (start 100.425 50.42) (end 62.73 50.42) (width 0.2) (layer "B.Cu") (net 13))
 (segment (start 54.5 42.434314) (end 62.434314 34.5) (width 0.2) (layer "B.Cu") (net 10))
 (segment (start 54.5 51) (end 54.5 42.434314) (width 0.2) (layer "B.Cu") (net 10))
 (segment (start 98.5 35) (end 62.5 35) (width 0.2) (layer "B.Cu") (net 11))
 (segment (start 62.5 35) (end 55 42.5) (width 0.2) (layer "B.Cu") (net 11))
 (segment (start 57.385 47.615) (end 62.73 52.96) (width 0.2) (layer "B.Cu") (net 12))
 (segment (start 62.73 52.96) (end 100.425 52.96) (width 0.2) (layer "B.Cu") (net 12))
 (segment (start 100.425 42.8) (end 99.34737 42.8) (width 0.2) (layer "F.Cu") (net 8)))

